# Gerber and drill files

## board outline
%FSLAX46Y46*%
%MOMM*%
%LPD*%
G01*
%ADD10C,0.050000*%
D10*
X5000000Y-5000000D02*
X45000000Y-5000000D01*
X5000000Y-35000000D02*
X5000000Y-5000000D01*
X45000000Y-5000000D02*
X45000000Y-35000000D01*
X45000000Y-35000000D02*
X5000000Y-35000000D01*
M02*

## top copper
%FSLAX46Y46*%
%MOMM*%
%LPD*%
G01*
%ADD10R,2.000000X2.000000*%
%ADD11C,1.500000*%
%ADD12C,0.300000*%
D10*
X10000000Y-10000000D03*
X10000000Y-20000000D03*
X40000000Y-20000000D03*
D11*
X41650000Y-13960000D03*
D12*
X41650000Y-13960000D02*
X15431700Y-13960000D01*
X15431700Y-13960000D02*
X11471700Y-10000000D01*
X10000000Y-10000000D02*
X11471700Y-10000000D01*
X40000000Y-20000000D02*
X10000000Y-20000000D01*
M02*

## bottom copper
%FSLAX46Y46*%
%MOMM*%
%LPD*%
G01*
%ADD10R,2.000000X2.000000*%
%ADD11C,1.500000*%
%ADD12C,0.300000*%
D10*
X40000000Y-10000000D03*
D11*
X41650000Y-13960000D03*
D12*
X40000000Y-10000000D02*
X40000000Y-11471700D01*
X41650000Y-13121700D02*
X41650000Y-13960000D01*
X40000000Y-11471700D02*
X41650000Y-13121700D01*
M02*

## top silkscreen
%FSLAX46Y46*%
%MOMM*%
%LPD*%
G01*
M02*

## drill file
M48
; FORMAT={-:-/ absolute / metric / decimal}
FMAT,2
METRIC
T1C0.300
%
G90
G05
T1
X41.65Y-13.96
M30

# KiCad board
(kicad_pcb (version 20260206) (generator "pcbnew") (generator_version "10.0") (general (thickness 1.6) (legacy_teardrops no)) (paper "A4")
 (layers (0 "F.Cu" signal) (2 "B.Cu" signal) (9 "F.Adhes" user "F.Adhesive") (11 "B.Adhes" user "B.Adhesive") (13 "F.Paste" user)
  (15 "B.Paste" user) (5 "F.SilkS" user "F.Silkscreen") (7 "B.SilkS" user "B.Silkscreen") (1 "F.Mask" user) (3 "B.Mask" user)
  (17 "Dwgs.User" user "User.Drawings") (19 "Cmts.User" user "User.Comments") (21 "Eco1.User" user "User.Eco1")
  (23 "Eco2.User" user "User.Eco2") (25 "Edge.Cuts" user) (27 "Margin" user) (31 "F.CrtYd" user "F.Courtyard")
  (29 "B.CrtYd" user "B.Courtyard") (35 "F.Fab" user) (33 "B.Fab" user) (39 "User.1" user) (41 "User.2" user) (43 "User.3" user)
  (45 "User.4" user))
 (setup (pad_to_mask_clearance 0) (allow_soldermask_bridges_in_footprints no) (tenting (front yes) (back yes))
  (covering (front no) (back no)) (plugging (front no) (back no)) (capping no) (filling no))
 (gr_line (start 5 5) (end 45 5) (stroke (width 0.05) (type default)) (layer "Edge.Cuts"))
 (gr_line (start 5 35) (end 5 5) (stroke (width 0.05) (type default)) (layer "Edge.Cuts"))
 (gr_line (start 45 5) (end 45 35) (stroke (width 0.05) (type default)) (layer "Edge.Cuts"))
 (gr_line (start 45 35) (end 5 35) (stroke (width 0.05) (type default)) (layer "Edge.Cuts"))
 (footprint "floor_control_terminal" (layer "F.Cu") (at 10 10)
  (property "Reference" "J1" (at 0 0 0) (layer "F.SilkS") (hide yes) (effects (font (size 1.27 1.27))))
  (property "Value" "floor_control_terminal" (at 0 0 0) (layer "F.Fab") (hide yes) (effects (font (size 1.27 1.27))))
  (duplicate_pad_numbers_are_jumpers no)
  (pad "1" smd rect (at 0 0) (size 2 2) (layers "F.Cu" "F.Paste" "F.Mask") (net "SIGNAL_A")))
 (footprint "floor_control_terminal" (layer "B.Cu") (at 40 10)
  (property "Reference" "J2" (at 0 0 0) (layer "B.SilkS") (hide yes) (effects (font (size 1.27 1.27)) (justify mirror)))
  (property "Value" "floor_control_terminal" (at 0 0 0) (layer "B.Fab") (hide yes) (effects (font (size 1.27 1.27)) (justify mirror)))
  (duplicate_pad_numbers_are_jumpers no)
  (pad "1" smd rect (at 0 0) (size 2 2) (layers "B.Cu" "B.Paste" "B.Mask") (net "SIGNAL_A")))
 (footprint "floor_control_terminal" (layer "F.Cu") (at 10 20)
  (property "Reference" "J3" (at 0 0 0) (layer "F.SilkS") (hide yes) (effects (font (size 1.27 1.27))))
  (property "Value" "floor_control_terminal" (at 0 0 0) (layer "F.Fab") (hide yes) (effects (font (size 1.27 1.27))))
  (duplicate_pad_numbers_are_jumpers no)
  (pad "1" smd rect (at 0 0) (size 2 2) (layers "F.Cu" "F.Paste" "F.Mask") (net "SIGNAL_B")))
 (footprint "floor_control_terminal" (layer "F.Cu") (at 40 20)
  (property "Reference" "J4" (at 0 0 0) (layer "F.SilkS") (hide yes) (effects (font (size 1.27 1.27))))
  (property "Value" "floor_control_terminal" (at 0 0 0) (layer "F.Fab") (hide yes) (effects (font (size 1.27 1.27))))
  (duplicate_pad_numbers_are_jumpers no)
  (pad "1" smd rect (at 0 0) (size 2 2) (layers "F.Cu" "F.Paste" "F.Mask") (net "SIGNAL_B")))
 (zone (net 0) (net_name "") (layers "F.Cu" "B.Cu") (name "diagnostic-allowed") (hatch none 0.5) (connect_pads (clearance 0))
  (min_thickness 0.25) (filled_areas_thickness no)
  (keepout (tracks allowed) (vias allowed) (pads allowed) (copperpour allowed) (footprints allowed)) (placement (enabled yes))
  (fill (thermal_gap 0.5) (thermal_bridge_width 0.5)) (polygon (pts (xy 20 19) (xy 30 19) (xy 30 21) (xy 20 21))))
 (segment (start 41.65 13.96) (end 15.4317 13.96) (width 0.3) (layer "F.Cu") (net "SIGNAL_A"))
 (segment (start 15.4317 13.96) (end 11.4717 10) (width 0.3) (layer "F.Cu") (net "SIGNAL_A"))
 (segment (start 10 10) (end 11.4717 10) (width 0.3) (layer "F.Cu") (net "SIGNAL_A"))
 (via (at 41.65 13.96) (size 1.5) (drill 0.3) (layers "F.Cu" "B.Cu") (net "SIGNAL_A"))
 (segment (start 40 10) (end 40 11.4717) (width 0.3) (layer "B.Cu") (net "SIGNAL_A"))
 (segment (start 41.65 13.1217) (end 41.65 13.96) (width 0.3) (layer "B.Cu") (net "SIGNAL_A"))
 (segment (start 40 11.4717) (end 41.65 13.1217) (width 0.3) (layer "B.Cu") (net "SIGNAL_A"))
 (segment (start 40 20) (end 10 20) (width 0.3) (layer "F.Cu") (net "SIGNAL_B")))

